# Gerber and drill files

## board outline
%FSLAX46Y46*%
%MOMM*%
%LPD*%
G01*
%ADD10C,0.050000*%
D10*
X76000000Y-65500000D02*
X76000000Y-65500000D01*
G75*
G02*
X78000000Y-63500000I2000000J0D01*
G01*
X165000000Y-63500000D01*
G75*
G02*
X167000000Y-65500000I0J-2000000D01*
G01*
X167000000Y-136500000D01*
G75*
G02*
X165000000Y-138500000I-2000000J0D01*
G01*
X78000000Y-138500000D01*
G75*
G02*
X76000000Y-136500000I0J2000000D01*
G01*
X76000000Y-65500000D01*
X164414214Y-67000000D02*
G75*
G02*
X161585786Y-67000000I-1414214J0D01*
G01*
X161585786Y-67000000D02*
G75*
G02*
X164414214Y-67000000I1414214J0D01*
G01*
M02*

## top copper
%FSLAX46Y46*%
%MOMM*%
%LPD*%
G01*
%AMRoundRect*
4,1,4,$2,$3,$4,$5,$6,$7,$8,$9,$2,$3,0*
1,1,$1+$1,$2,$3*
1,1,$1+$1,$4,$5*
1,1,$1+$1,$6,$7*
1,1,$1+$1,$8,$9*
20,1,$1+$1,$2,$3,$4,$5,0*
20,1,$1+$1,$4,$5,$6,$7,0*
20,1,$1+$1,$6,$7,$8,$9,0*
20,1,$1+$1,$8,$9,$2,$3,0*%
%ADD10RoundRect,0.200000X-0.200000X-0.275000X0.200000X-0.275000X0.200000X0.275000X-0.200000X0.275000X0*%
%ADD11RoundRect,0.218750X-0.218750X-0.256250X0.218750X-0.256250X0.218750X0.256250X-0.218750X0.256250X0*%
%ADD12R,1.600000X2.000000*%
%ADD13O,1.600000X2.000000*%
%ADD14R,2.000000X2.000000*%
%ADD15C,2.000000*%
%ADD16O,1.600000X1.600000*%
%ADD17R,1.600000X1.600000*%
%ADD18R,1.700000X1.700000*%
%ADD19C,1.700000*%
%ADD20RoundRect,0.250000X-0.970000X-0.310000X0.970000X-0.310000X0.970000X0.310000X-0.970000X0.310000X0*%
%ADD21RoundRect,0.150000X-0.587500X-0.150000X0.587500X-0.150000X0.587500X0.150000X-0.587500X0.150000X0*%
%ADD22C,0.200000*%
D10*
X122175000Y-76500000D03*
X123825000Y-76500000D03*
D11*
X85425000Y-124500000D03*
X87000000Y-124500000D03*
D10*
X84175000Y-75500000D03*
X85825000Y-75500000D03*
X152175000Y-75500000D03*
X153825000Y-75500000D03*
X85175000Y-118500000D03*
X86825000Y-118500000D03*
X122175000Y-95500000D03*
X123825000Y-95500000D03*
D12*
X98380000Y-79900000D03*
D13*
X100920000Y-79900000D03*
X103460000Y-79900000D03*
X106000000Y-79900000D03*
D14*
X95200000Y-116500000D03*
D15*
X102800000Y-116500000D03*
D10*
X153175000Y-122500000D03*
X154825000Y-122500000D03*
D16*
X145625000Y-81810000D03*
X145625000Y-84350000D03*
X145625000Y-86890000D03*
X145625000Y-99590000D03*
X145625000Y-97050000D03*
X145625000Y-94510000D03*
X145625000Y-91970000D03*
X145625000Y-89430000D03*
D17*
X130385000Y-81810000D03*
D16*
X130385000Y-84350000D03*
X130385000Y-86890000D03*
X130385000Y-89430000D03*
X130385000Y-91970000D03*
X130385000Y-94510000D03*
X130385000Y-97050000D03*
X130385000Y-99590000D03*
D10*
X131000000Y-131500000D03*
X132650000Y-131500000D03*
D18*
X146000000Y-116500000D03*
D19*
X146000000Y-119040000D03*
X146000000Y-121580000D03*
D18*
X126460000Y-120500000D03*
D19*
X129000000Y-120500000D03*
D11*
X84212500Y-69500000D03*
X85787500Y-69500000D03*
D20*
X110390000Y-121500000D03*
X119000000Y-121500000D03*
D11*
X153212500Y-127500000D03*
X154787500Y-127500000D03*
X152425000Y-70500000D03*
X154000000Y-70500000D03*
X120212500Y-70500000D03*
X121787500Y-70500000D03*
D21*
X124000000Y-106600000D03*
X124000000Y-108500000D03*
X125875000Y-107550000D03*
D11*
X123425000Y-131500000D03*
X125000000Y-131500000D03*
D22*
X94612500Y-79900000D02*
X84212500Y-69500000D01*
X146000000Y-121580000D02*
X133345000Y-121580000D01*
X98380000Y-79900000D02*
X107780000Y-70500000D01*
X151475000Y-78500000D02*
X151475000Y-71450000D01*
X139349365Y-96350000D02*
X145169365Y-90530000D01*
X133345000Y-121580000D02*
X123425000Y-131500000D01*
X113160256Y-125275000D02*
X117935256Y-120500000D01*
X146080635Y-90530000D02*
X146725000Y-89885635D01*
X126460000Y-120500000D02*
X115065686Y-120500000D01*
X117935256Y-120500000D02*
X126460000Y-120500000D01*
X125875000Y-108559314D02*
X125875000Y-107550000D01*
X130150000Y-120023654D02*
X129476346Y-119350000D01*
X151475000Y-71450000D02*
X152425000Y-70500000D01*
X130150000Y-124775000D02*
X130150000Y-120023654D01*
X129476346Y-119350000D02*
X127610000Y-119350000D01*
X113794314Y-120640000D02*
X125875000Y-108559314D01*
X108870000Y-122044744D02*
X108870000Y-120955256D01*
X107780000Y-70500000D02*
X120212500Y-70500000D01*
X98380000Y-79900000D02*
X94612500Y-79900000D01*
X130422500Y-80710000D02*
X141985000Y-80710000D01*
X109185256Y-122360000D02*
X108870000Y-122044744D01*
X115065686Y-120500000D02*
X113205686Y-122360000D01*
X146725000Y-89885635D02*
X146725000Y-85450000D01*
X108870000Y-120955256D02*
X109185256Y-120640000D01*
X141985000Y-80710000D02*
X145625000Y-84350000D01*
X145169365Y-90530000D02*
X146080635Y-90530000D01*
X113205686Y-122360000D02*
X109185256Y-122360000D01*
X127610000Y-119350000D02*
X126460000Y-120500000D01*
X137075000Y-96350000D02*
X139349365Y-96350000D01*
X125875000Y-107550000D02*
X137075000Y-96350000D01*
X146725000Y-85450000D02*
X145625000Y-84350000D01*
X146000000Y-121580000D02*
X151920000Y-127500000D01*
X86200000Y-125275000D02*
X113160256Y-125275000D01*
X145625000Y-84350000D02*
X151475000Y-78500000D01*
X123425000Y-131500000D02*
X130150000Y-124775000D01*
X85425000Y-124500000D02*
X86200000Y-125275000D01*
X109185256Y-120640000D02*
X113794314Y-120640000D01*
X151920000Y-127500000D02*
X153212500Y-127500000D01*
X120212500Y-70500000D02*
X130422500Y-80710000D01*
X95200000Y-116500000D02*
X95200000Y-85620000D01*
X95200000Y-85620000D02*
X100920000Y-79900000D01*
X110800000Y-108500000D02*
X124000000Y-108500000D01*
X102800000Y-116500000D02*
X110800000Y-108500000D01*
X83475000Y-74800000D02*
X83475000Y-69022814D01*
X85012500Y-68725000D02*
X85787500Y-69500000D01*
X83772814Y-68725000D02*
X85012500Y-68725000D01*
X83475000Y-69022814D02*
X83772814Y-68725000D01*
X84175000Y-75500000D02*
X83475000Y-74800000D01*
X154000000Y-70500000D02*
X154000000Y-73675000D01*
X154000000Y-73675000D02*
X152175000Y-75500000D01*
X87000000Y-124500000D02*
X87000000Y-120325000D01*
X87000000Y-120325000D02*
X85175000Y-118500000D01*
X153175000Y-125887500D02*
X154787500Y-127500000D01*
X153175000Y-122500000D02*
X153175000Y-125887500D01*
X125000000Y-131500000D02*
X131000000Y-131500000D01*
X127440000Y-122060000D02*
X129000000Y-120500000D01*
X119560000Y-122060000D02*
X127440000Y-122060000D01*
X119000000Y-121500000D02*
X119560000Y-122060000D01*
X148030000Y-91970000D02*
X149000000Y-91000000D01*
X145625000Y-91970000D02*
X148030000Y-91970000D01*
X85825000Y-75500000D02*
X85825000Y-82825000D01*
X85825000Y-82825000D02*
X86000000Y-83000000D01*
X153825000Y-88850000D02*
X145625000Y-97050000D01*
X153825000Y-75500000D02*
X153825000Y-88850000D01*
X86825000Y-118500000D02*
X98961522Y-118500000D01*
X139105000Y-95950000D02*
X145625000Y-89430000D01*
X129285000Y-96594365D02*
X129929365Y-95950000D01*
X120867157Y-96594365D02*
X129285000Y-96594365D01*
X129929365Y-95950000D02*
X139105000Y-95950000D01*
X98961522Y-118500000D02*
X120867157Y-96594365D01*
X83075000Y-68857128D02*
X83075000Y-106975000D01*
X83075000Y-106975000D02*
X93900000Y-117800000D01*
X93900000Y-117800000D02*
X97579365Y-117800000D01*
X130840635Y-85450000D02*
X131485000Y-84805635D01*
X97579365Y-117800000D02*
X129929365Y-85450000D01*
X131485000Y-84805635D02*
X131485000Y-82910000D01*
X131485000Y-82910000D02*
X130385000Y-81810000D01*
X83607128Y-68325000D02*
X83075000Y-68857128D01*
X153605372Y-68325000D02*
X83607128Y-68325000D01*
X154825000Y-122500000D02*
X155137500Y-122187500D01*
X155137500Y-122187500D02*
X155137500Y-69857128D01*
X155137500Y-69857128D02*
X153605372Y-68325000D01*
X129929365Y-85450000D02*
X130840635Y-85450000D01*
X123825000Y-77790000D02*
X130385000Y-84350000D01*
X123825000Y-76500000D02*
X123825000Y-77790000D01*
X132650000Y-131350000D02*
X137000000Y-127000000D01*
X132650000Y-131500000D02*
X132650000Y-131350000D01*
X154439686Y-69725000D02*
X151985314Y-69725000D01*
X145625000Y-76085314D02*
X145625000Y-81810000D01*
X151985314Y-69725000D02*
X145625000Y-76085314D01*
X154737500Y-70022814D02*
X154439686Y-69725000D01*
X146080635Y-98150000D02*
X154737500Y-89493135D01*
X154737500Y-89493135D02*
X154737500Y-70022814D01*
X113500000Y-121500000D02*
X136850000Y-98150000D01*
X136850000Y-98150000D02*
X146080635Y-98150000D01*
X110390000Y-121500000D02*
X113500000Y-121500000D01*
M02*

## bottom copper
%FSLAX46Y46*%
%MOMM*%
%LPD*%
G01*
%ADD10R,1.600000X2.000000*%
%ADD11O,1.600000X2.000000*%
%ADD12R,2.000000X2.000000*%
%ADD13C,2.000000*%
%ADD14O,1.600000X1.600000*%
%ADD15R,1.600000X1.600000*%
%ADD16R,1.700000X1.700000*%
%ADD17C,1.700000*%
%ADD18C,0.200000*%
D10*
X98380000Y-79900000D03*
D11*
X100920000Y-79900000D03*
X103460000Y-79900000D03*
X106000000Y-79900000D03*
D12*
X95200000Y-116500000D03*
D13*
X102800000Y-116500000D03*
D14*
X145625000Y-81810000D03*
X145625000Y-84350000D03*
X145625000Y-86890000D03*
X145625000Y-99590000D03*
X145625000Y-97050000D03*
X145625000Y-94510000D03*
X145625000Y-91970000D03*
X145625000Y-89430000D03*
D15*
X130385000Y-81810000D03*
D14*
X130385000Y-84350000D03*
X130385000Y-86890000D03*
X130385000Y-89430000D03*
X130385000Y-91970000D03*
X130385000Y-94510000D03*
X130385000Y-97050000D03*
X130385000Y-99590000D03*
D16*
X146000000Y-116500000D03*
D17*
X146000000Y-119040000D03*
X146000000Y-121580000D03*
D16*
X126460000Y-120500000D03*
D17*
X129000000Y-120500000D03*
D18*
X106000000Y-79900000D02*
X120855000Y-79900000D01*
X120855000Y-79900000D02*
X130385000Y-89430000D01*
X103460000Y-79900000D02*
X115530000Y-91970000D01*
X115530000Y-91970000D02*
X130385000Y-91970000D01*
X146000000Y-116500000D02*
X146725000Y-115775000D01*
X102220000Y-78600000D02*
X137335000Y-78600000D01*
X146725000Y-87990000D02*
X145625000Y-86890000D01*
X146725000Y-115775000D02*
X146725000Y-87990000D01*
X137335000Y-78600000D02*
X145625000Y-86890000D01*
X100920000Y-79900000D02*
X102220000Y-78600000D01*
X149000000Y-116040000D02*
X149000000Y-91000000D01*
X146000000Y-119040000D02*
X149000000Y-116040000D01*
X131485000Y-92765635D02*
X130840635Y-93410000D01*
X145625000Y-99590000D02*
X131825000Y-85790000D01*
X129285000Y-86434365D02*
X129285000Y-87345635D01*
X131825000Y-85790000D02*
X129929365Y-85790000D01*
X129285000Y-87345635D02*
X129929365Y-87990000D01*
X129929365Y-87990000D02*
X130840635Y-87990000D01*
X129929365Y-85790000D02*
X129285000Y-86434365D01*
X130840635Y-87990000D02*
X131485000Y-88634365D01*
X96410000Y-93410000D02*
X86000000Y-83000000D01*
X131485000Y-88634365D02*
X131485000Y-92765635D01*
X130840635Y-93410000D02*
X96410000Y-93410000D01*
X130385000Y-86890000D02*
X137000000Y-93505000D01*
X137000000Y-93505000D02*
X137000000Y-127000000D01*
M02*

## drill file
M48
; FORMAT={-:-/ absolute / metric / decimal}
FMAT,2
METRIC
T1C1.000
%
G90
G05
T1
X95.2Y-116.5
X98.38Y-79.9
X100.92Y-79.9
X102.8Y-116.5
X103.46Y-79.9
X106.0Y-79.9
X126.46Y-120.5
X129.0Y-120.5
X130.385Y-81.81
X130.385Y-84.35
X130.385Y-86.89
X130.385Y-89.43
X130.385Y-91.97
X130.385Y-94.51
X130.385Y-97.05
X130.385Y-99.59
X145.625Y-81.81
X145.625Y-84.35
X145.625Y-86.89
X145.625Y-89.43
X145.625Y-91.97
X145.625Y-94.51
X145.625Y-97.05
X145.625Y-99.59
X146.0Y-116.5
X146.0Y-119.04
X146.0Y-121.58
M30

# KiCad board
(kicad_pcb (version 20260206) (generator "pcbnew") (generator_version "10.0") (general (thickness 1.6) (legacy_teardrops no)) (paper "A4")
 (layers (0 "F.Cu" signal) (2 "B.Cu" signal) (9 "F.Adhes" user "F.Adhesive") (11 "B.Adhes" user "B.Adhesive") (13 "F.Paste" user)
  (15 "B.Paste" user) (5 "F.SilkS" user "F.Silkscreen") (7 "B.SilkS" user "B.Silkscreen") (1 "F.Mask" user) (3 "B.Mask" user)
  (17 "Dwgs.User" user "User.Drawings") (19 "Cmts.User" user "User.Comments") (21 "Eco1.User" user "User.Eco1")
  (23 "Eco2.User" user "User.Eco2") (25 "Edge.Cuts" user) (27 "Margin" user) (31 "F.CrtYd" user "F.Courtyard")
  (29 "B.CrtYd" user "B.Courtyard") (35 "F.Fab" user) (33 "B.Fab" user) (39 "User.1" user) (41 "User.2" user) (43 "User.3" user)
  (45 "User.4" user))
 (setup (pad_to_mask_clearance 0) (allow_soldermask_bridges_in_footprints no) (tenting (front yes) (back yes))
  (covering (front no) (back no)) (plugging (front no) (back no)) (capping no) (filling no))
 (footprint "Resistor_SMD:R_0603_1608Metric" (layer "F.Cu") (at 123 76.5)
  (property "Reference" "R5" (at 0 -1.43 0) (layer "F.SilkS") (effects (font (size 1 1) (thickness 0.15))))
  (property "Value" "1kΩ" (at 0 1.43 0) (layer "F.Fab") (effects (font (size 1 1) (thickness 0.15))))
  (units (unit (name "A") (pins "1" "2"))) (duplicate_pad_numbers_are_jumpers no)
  (pad "1" smd roundrect (at -0.825 0) (size 0.8 0.95) (layers "F.Cu" "F.Mask" "F.Paste") (roundrect_rratio 0.25) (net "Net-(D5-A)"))
  (pad "2" smd roundrect (at 0.825 0) (size 0.8 0.95) (layers "F.Cu" "F.Mask" "F.Paste") (roundrect_rratio 0.25) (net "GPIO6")))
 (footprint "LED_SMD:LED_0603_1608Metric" (layer "F.Cu") (at 86.2125 124.5)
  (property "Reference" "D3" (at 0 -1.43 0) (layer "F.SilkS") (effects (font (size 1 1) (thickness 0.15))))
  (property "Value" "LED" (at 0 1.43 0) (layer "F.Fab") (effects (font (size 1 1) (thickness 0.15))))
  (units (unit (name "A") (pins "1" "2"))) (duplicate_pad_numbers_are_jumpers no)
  (pad "1" smd roundrect (at -0.7875 0) (size 0.875 0.95) (layers "F.Cu" "F.Mask" "F.Paste") (roundrect_rratio 0.25) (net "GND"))
  (pad "2" smd roundrect (at 0.7875 0) (size 0.875 0.95) (layers "F.Cu" "F.Mask" "F.Paste") (roundrect_rratio 0.25) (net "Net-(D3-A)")))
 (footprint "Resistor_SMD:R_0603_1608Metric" (layer "F.Cu") (at 85 75.5)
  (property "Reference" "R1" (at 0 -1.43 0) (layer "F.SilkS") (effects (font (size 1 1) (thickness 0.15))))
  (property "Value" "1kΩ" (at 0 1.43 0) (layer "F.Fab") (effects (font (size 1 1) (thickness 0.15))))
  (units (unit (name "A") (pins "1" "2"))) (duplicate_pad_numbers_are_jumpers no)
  (pad "1" smd roundrect (at -0.825 0) (size 0.8 0.95) (layers "F.Cu" "F.Mask" "F.Paste") (roundrect_rratio 0.25) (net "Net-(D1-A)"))
  (pad "2" smd roundrect (at 0.825 0) (size 0.8 0.95) (layers "F.Cu" "F.Mask" "F.Paste") (roundrect_rratio 0.25) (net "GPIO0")))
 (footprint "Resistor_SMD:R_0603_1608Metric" (layer "F.Cu") (at 153 75.5)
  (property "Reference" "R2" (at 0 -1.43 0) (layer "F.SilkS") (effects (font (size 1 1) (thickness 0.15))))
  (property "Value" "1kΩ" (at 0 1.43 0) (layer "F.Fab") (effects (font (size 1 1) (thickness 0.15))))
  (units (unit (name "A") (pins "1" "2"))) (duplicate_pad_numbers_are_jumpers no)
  (pad "1" smd roundrect (at -0.825 0) (size 0.8 0.95) (layers "F.Cu" "F.Mask" "F.Paste") (roundrect_rratio 0.25) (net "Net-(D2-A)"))
  (pad "2" smd roundrect (at 0.825 0) (size 0.8 0.95) (layers "F.Cu" "F.Mask" "F.Paste") (roundrect_rratio 0.25) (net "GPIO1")))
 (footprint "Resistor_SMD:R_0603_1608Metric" (layer "F.Cu") (at 86 118.5)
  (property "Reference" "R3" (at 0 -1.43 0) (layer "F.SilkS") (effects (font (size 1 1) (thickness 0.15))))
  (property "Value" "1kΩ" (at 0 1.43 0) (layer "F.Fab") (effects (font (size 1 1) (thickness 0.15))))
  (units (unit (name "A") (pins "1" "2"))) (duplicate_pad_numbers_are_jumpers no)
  (pad "1" smd roundrect (at -0.825 0) (size 0.8 0.95) (layers "F.Cu" "F.Mask" "F.Paste") (roundrect_rratio 0.25) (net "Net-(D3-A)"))
  (pad "2" smd roundrect (at 0.825 0) (size 0.8 0.95) (layers "F.Cu" "F.Mask" "F.Paste") (roundrect_rratio 0.25) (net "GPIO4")))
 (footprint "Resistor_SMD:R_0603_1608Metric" (layer "F.Cu") (at 123 95.5)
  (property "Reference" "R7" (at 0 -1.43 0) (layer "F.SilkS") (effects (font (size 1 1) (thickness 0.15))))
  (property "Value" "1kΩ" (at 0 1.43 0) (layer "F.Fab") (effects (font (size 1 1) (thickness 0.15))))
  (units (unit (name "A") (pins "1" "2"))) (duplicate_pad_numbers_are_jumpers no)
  (pad "1" smd roundrect (at -0.825 0) (size 0.8 0.95) (layers "F.Cu" "F.Mask" "F.Paste") (roundrect_rratio 0.25) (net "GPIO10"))
  (pad "2" smd roundrect (at 0.825 0) (size 0.8 0.95) (layers "F.Cu" "F.Mask" "F.Paste") (roundrect_rratio 0.25) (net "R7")))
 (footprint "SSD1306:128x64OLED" (layer "F.Cu") (at 102 90.5)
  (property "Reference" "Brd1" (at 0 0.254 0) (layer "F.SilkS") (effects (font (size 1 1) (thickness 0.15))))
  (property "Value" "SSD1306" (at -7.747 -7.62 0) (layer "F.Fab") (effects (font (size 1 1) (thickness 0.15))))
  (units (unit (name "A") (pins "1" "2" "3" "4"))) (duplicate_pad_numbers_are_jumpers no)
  (pad "1" thru_hole rect (at -3.62 -10.6 90) (size 2 1.6) (drill 1) (layers "*.Cu" "*.Mask") (remove_unused_layers no) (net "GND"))
  (pad "2" thru_hole oval (at -1.08 -10.6 90) (size 2 1.6) (drill 1) (layers "*.Cu" "*.Mask") (remove_unused_layers no) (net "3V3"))
  (pad "3" thru_hole oval (at 1.46 -10.6 90) (size 2 1.6) (drill 1) (layers "*.Cu" "*.Mask") (remove_unused_layers no) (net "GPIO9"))
  (pad "4" thru_hole oval (at 4 -10.6 90) (size 2 1.6) (drill 1) (layers "*.Cu" "*.Mask") (remove_unused_layers no) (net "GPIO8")))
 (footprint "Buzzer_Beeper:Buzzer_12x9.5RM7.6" (layer "F.Cu") (at 95.2 116.5)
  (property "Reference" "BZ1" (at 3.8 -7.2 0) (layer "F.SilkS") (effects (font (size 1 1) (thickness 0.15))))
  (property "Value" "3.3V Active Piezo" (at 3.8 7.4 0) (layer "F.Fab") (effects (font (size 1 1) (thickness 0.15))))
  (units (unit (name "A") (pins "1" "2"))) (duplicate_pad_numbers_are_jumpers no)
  (pad "1" thru_hole rect (at 0 0) (size 2 2) (drill 1) (layers "*.Cu" "*.Mask") (remove_unused_layers no) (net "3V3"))
  (pad "2" thru_hole circle (at 7.6 0) (size 2 2) (drill 1) (layers "*.Cu" "*.Mask") (remove_unused_layers no) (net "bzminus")))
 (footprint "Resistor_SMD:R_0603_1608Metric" (layer "F.Cu") (at 154 122.5)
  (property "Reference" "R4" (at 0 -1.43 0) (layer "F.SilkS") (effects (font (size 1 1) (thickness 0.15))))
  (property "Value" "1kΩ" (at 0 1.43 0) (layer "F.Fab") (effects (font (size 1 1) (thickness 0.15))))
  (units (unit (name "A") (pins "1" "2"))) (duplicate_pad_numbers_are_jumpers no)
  (pad "1" smd roundrect (at -0.825 0) (size 0.8 0.95) (layers "F.Cu" "F.Mask" "F.Paste") (roundrect_rratio 0.25) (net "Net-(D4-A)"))
  (pad "2" smd roundrect (at 0.825 0) (size 0.8 0.95) (layers "F.Cu" "F.Mask" "F.Paste") (roundrect_rratio 0.25) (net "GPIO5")))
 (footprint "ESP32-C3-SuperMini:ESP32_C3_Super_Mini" (layer "F.Cu") (at 130.385 81.81)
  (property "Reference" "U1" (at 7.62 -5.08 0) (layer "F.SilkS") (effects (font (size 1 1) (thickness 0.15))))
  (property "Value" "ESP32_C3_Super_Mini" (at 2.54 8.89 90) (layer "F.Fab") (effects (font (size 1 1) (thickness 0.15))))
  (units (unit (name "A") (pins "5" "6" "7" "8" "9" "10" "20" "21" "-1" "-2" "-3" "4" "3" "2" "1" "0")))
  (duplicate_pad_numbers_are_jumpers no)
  (pad "-1" thru_hole oval (at 15.24 0) (size 1.6 1.6) (drill 1) (layers "*.Cu" "*.Mask") (remove_unused_layers no) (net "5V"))
  (pad "-2" thru_hole oval (at 15.24 2.54) (size 1.6 1.6) (drill 1) (layers "*.Cu" "*.Mask") (remove_unused_layers no) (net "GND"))
  (pad "-3" thru_hole oval (at 15.24 5.08) (size 1.6 1.6) (drill 1) (layers "*.Cu" "*.Mask") (remove_unused_layers no) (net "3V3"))
  (pad "0" thru_hole oval (at 15.24 17.78) (size 1.6 1.6) (drill 1) (layers "*.Cu" "*.Mask") (remove_unused_layers no) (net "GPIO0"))
  (pad "1" thru_hole oval (at 15.24 15.24) (size 1.6 1.6) (drill 1) (layers "*.Cu" "*.Mask") (remove_unused_layers no) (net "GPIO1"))
  (pad "2" thru_hole oval (at 15.24 12.7) (size 1.6 1.6) (drill 1) (layers "*.Cu" "*.Mask") (remove_unused_layers no)
   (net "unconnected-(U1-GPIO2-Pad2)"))
  (pad "3" thru_hole oval (at 15.24 10.16) (size 1.6 1.6) (drill 1) (layers "*.Cu" "*.Mask") (remove_unused_layers no) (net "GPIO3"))
  (pad "4" thru_hole oval (at 15.24 7.62) (size 1.6 1.6) (drill 1) (layers "*.Cu" "*.Mask") (remove_unused_layers no) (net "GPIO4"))
  (pad "5" thru_hole rect (at 0 0) (size 1.6 1.6) (drill 1) (layers "*.Cu" "*.Mask") (remove_unused_layers no) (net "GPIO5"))
  (pad "6" thru_hole oval (at 0 2.54) (size 1.6 1.6) (drill 1) (layers "*.Cu" "*.Mask") (remove_unused_layers no) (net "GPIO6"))
  (pad "7" thru_hole oval (at 0 5.08) (size 1.6 1.6) (drill 1) (layers "*.Cu" "*.Mask") (remove_unused_layers no) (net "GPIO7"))
  (pad "8" thru_hole oval (at 0 7.62) (size 1.6 1.6) (drill 1) (layers "*.Cu" "*.Mask") (remove_unused_layers no) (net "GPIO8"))
  (pad "9" thru_hole oval (at 0 10.16) (size 1.6 1.6) (drill 1) (layers "*.Cu" "*.Mask") (remove_unused_layers no) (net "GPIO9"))
  (pad "10" thru_hole oval (at 0 12.7) (size 1.6 1.6) (drill 1) (layers "*.Cu" "*.Mask") (remove_unused_layers no) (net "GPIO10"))
  (pad "20" thru_hole oval (at 0 15.24) (size 1.6 1.6) (drill 1) (layers "*.Cu" "*.Mask") (remove_unused_layers no)
   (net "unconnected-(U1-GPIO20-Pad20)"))
  (pad "21" thru_hole oval (at 0 17.78) (size 1.6 1.6) (drill 1) (layers "*.Cu" "*.Mask") (remove_unused_layers no)
   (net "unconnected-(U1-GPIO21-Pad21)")))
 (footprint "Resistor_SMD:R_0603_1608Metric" (layer "F.Cu") (at 131.825 131.5)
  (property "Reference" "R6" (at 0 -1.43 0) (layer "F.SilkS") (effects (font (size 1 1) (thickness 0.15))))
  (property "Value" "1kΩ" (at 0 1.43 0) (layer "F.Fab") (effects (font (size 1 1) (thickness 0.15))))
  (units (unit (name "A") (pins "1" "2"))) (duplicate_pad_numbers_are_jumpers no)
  (pad "1" smd roundrect (at -0.825 0) (size 0.8 0.95) (layers "F.Cu" "F.Mask" "F.Paste") (roundrect_rratio 0.25) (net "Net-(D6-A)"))
  (pad "2" smd roundrect (at 0.825 0) (size 0.8 0.95) (layers "F.Cu" "F.Mask" "F.Paste") (roundrect_rratio 0.25) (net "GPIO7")))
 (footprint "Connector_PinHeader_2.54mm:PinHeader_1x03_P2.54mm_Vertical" (layer "F.Cu") (at 146 116.5)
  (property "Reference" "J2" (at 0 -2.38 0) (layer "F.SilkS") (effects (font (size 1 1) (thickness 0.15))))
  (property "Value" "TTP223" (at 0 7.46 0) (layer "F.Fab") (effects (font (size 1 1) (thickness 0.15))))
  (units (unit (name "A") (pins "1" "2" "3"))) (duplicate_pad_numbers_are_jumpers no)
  (pad "1" thru_hole rect (at 0 0) (size 1.7 1.7) (drill 1) (layers "*.Cu" "*.Mask") (remove_unused_layers no) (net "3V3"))
  (pad "2" thru_hole circle (at 0 2.54) (size 1.7 1.7) (drill 1) (layers "*.Cu" "*.Mask") (remove_unused_layers no) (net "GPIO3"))
  (pad "3" thru_hole circle (at 0 5.08) (size 1.7 1.7) (drill 1) (layers "*.Cu" "*.Mask") (remove_unused_layers no) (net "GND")))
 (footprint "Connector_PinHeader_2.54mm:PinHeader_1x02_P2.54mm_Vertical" (layer "F.Cu") (at 126.46 120.5 90)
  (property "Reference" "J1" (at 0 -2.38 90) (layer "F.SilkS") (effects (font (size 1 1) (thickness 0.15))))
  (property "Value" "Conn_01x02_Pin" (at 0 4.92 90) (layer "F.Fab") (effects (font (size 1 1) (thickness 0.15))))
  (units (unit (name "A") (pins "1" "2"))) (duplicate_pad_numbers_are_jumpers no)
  (pad "1" thru_hole rect (at 0 0 90) (size 1.7 1.7) (drill 1) (layers "*.Cu" "*.Mask") (remove_unused_layers no) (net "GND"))
  (pad "2" thru_hole circle (at 0 2.54 90) (size 1.7 1.7) (drill 1) (layers "*.Cu" "*.Mask") (remove_unused_layers no)
   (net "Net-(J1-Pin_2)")))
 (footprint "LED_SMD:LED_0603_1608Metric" (layer "F.Cu") (at 85 69.5)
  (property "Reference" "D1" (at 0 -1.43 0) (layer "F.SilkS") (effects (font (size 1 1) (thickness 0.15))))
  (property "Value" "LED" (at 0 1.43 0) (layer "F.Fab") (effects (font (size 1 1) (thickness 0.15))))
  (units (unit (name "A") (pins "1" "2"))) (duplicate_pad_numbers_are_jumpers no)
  (pad "1" smd roundrect (at -0.7875 0) (size 0.875 0.95) (layers "F.Cu" "F.Mask" "F.Paste") (roundrect_rratio 0.25) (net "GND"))
  (pad "2" smd roundrect (at 0.7875 0) (size 0.875 0.95) (layers "F.Cu" "F.Mask" "F.Paste") (roundrect_rratio 0.25) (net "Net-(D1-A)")))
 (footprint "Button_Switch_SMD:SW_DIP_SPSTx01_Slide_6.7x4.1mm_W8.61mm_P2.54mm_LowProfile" (layer "F.Cu") (at 114.695 121.5)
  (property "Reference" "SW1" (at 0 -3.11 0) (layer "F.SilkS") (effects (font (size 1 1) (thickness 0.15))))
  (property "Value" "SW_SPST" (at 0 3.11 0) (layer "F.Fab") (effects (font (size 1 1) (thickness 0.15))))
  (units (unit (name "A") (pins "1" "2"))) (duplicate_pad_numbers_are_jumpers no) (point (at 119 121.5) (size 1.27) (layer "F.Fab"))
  (pad "1" smd roundrect (at -4.305 0) (size 2.44 1.12) (layers "F.Cu" "F.Mask" "F.Paste") (roundrect_rratio 0.223214) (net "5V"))
  (pad "2" smd roundrect (at 4.305 0) (size 2.44 1.12) (layers "F.Cu" "F.Mask" "F.Paste") (roundrect_rratio 0.223214) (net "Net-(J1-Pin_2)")))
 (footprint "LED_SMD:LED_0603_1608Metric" (layer "F.Cu") (at 154 127.5)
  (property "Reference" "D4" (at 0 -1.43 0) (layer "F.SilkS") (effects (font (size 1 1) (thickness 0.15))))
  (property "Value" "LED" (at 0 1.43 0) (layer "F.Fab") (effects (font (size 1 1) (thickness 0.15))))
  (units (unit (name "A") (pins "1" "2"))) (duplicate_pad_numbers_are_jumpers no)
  (pad "1" smd roundrect (at -0.7875 0) (size 0.875 0.95) (layers "F.Cu" "F.Mask" "F.Paste") (roundrect_rratio 0.25) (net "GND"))
  (pad "2" smd roundrect (at 0.7875 0) (size 0.875 0.95) (layers "F.Cu" "F.Mask" "F.Paste") (roundrect_rratio 0.25) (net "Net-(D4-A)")))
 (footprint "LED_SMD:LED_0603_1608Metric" (layer "F.Cu") (at 153.2125 70.5)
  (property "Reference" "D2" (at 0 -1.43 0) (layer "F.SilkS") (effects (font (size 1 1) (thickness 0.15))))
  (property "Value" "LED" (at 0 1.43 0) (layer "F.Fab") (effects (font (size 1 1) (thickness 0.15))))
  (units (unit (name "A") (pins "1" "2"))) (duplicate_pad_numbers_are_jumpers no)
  (pad "1" smd roundrect (at -0.7875 0) (size 0.875 0.95) (layers "F.Cu" "F.Mask" "F.Paste") (roundrect_rratio 0.25) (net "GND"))
  (pad "2" smd roundrect (at 0.7875 0) (size 0.875 0.95) (layers "F.Cu" "F.Mask" "F.Paste") (roundrect_rratio 0.25) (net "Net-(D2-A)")))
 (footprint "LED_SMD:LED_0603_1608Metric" (layer "F.Cu") (at 121 70.5)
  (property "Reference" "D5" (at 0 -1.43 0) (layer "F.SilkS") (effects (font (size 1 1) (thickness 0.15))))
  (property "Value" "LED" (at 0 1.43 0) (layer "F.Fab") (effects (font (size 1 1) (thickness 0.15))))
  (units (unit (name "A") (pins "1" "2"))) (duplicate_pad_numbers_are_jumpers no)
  (pad "1" smd roundrect (at -0.7875 0) (size 0.875 0.95) (layers "F.Cu" "F.Mask" "F.Paste") (roundrect_rratio 0.25) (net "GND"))
  (pad "2" smd roundrect (at 0.7875 0) (size 0.875 0.95) (layers "F.Cu" "F.Mask" "F.Paste") (roundrect_rratio 0.25) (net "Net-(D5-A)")))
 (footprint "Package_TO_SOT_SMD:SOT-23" (layer "F.Cu") (at 124.9375 107.55)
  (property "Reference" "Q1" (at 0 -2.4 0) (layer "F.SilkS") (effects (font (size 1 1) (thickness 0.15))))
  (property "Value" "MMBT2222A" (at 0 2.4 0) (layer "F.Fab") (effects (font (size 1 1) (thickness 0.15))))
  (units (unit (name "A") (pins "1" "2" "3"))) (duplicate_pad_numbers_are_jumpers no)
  (pad "1" smd roundrect (at -0.9375 -0.95) (size 1.475 0.6) (layers "F.Cu" "F.Mask" "F.Paste") (roundrect_rratio 0.25) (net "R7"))
  (pad "2" smd roundrect (at -0.9375 0.95) (size 1.475 0.6) (layers "F.Cu" "F.Mask" "F.Paste") (roundrect_rratio 0.25) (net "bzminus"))
  (pad "3" smd roundrect (at 0.9375 0) (size 1.475 0.6) (layers "F.Cu" "F.Mask" "F.Paste") (roundrect_rratio 0.25) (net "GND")))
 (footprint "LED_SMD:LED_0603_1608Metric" (layer "F.Cu") (at 124.2125 131.5)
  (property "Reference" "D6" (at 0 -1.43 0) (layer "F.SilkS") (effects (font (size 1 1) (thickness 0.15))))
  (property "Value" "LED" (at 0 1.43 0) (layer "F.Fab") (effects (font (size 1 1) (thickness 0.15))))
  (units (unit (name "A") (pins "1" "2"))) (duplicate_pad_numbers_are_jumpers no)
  (pad "1" smd roundrect (at -0.7875 0) (size 0.875 0.95) (layers "F.Cu" "F.Mask" "F.Paste") (roundrect_rratio 0.25) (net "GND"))
  (pad "2" smd roundrect (at 0.7875 0) (size 0.875 0.95) (layers "F.Cu" "F.Mask" "F.Paste") (roundrect_rratio 0.25) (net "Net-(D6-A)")))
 (gr_rect (start 76 63.5) (end 167 138.5) (radius 2) (stroke (width 0.05) (type default)) (fill no) (layer "Edge.Cuts"))
 (gr_circle (center 163 67) (end 164 68) (stroke (width 0.05) (type default)) (fill no) (layer "Edge.Cuts"))
 (segment (start 94.6125 79.9) (end 84.2125 69.5) (width 0.2) (layer "F.Cu") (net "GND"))
 (segment (start 146 121.58) (end 133.345 121.58) (width 0.2) (layer "F.Cu") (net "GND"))
 (segment (start 98.38 79.9) (end 107.78 70.5) (width 0.2) (layer "F.Cu") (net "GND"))
 (segment (start 151.475 78.5) (end 151.475 71.45) (width 0.2) (layer "F.Cu") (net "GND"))
 (segment (start 139.349365 96.35) (end 145.169365 90.53) (width 0.2) (layer "F.Cu") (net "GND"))
 (segment (start 133.345 121.58) (end 123.425 131.5) (width 0.2) (layer "F.Cu") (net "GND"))
 (segment (start 113.160256 125.275) (end 117.935256 120.5) (width 0.2) (layer "F.Cu") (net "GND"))
 (segment (start 146.080635 90.53) (end 146.725 89.885635) (width 0.2) (layer "F.Cu") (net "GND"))
 (segment (start 126.46 120.5) (end 115.065686 120.5) (width 0.2) (layer "F.Cu") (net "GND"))
 (segment (start 117.935256 120.5) (end 126.46 120.5) (width 0.2) (layer "F.Cu") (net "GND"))
 (segment (start 125.875 108.559314) (end 125.875 107.55) (width 0.2) (layer "F.Cu") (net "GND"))
 (segment (start 130.15 120.023654) (end 129.476346 119.35) (width 0.2) (layer "F.Cu") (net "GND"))
 (segment (start 151.475 71.45) (end 152.425 70.5) (width 0.2) (layer "F.Cu") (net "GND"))
 (segment (start 130.15 124.775) (end 130.15 120.023654) (width 0.2) (layer "F.Cu") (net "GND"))
 (segment (start 129.476346 119.35) (end 127.61 119.35) (width 0.2) (layer "F.Cu") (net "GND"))
 (segment (start 113.794314 120.64) (end 125.875 108.559314) (width 0.2) (layer "F.Cu") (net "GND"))
 (segment (start 108.87 122.044744) (end 108.87 120.955256) (width 0.2) (layer "F.Cu") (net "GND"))
 (segment (start 107.78 70.5) (end 120.2125 70.5) (width 0.2) (layer "F.Cu") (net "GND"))
 (segment (start 98.38 79.9) (end 94.6125 79.9) (width 0.2) (layer "F.Cu") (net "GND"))
 (segment (start 130.4225 80.71) (end 141.985 80.71) (width 0.2) (layer "F.Cu") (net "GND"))
 (segment (start 109.185256 122.36) (end 108.87 122.044744) (width 0.2) (layer "F.Cu") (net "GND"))
 (segment (start 115.065686 120.5) (end 113.205686 122.36) (width 0.2) (layer "F.Cu") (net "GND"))
 (segment (start 146.725 89.885635) (end 146.725 85.45) (width 0.2) (layer "F.Cu") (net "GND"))
 (segment (start 108.87 120.955256) (end 109.185256 120.64) (width 0.2) (layer "F.Cu") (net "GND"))
 (segment (start 141.985 80.71) (end 145.625 84.35) (width 0.2) (layer "F.Cu") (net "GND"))
 (segment (start 145.169365 90.53) (end 146.080635 90.53) (width 0.2) (layer "F.Cu") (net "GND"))
 (segment (start 113.205686 122.36) (end 109.185256 122.36) (width 0.2) (layer "F.Cu") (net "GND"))
 (segment (start 127.61 119.35) (end 126.46 120.5) (width 0.2) (layer "F.Cu") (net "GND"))
 (segment (start 137.075 96.35) (end 139.349365 96.35) (width 0.2) (layer "F.Cu") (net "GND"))
 (segment (start 125.875 107.55) (end 137.075 96.35) (width 0.2) (layer "F.Cu") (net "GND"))
 (segment (start 146.725 85.45) (end 145.625 84.35) (width 0.2) (layer "F.Cu") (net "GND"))
 (segment (start 146 121.58) (end 151.92 127.5) (width 0.2) (layer "F.Cu") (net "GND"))
 (segment (start 86.2 125.275) (end 113.160256 125.275) (width 0.2) (layer "F.Cu") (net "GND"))
 (segment (start 145.625 84.35) (end 151.475 78.5) (width 0.2) (layer "F.Cu") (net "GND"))
 (segment (start 123.425 131.5) (end 130.15 124.775) (width 0.2) (layer "F.Cu") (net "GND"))
 (segment (start 85.425 124.5) (end 86.2 125.275) (width 0.2) (layer "F.Cu") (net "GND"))
 (segment (start 109.185256 120.64) (end 113.794314 120.64) (width 0.2) (layer "F.Cu") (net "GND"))
 (segment (start 151.92 127.5) (end 153.2125 127.5) (width 0.2) (layer "F.Cu") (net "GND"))
 (segment (start 120.2125 70.5) (end 130.4225 80.71) (width 0.2) (layer "F.Cu") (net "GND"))
 (segment (start 106 79.9) (end 120.855 79.9) (width 0.2) (layer "B.Cu") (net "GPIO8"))
 (segment (start 120.855 79.9) (end 130.385 89.43) (width 0.2) (layer "B.Cu") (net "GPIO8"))
 (segment (start 103.46 79.9) (end 115.53 91.97) (width 0.2) (layer "B.Cu") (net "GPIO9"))
 (segment (start 115.53 91.97) (end 130.385 91.97) (width 0.2) (layer "B.Cu") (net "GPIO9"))
 (segment (start 95.2 116.5) (end 95.2 85.62) (width 0.2) (layer "F.Cu") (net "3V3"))
 (segment (start 95.2 85.62) (end 100.92 79.9) (width 0.2) (layer "F.Cu") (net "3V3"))
 (segment (start 146 116.5) (end 146.725 115.775) (width 0.2) (layer "B.Cu") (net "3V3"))
 (segment (start 102.22 78.6) (end 137.335 78.6) (width 0.2) (layer "B.Cu") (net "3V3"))
 (segment (start 146.725 87.99) (end 145.625 86.89) (width 0.2) (layer "B.Cu") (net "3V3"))
 (segment (start 146.725 115.775) (end 146.725 87.99) (width 0.2) (layer "B.Cu") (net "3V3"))
 (segment (start 137.335 78.6) (end 145.625 86.89) (width 0.2) (layer "B.Cu") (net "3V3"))
 (segment (start 100.92 79.9) (end 102.22 78.6) (width 0.2) (layer "B.Cu") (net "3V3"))
 (segment (start 110.8 108.5) (end 124 108.5) (width 0.2) (layer "F.Cu") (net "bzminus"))
 (segment (start 102.8 116.5) (end 110.8 108.5) (width 0.2) (layer "F.Cu") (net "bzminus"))
 (segment (start 83.475 74.8) (end 83.475 69.022814) (width 0.2) (layer "F.Cu") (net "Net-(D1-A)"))
 (segment (start 85.0125 68.725) (end 85.7875 69.5) (width 0.2) (layer "F.Cu") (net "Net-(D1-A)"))
 (segment (start 83.772814 68.725) (end 85.0125 68.725) (width 0.2) (layer "F.Cu") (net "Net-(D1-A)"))
 (segment (start 83.475 69.022814) (end 83.772814 68.725) (width 0.2) (layer "F.Cu") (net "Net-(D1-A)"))
 (segment (start 84.175 75.5) (end 83.475 74.8) (width 0.2) (layer "F.Cu") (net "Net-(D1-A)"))
 (segment (start 154 70.5) (end 154 73.675) (width 0.2) (layer "F.Cu") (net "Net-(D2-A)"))
 (segment (start 154 73.675) (end 152.175 75.5) (width 0.2) (layer "F.Cu") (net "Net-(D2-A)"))
 (segment (start 87 124.5) (end 87 120.325) (width 0.2) (layer "F.Cu") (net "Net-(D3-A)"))
 (segment (start 87 120.325) (end 85.175 118.5) (width 0.2) (layer "F.Cu") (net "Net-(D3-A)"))
 (segment (start 153.175 125.8875) (end 154.7875 127.5) (width 0.2) (layer "F.Cu") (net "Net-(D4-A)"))
 (segment (start 153.175 122.5) (end 153.175 125.8875) (width 0.2) (layer "F.Cu") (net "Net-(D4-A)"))
 (segment (start 125 131.5) (end 131 131.5) (width 0.2) (layer "F.Cu") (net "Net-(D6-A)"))
 (segment (start 127.44 122.06) (end 129 120.5) (width 0.2) (layer "F.Cu") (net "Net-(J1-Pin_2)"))
 (segment (start 119.56 122.06) (end 127.44 122.06) (width 0.2) (layer "F.Cu") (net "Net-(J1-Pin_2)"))
 (segment (start 119 121.5) (end 119.56 122.06) (width 0.2) (layer "F.Cu") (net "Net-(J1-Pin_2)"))
 (segment (start 148.03 91.97) (end 149 91) (width 0.2) (layer "F.Cu") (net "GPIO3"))
 (segment (start 145.625 91.97) (end 148.03 91.97) (width 0.2) (layer "F.Cu") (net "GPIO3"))
 (segment (start 149 116.04) (end 149 91) (width 0.2) (layer "B.Cu") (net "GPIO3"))
 (segment (start 146 119.04) (end 149 116.04) (width 0.2) (layer "B.Cu") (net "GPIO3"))
 (segment (start 85.825 75.5) (end 85.825 82.825) (width 0.2) (layer "F.Cu") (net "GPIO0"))
 (segment (start 85.825 82.825) (end 86 83) (width 0.2) (layer "F.Cu") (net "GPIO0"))
 (segment (start 131.485 92.765635) (end 130.840635 93.41) (width 0.2) (layer "B.Cu") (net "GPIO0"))
 (segment (start 145.625 99.59) (end 131.825 85.79) (width 0.2) (layer "B.Cu") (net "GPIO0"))
 (segment (start 129.285 86.434365) (end 129.285 87.345635) (width 0.2) (layer "B.Cu") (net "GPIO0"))
 (segment (start 131.825 85.79) (end 129.929365 85.79) (width 0.2) (layer "B.Cu") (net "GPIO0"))
 (segment (start 129.285 87.345635) (end 129.929365 87.99) (width 0.2) (layer "B.Cu") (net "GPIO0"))
 (segment (start 129.929365 87.99) (end 130.840635 87.99) (width 0.2) (layer "B.Cu") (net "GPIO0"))
 (segment (start 129.929365 85.79) (end 129.285 86.434365) (width 0.2) (layer "B.Cu") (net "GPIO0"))
 (segment (start 130.840635 87.99) (end 131.485 88.634365) (width 0.2) (layer "B.Cu") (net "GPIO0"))
 (segment (start 96.41 93.41) (end 86 83) (width 0.2) (layer "B.Cu") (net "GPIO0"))
 (segment (start 131.485 88.634365) (end 131.485 92.765635) (width 0.2) (layer "B.Cu") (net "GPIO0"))
 (segment (start 130.840635 93.41) (end 96.41 93.41) (width 0.2) (layer "B.Cu") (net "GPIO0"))
 (segment (start 153.825 88.85) (end 145.625 97.05) (width 0.2) (layer "F.Cu") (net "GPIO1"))
 (segment (start 153.825 75.5) (end 153.825 88.85) (width 0.2) (layer "F.Cu") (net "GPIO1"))
 (segment (start 86.825 118.5) (end 98.961522 118.5) (width 0.2) (layer "F.Cu") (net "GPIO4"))
 (segment (start 139.105 95.95) (end 145.625 89.43) (width 0.2) (layer "F.Cu") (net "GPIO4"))
 (segment (start 129.285 96.594365) (end 129.929365 95.95) (width 0.2) (layer "F.Cu") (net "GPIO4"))
 (segment (start 120.867157 96.594365) (end 129.285 96.594365) (width 0.2) (layer "F.Cu") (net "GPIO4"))
 (segment (start 129.929365 95.95) (end 139.105 95.95) (width 0.2) (layer "F.Cu") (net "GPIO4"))
 (segment (start 98.961522 118.5) (end 120.867157 96.594365) (width 0.2) (layer "F.Cu") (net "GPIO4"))
 (segment (start 83.075 68.857128) (end 83.075 106.975) (width 0.2) (layer "F.Cu") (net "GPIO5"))
 (segment (start 83.075 106.975) (end 93.9 117.8) (width 0.2) (layer "F.Cu") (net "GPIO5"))
 (segment (start 93.9 117.8) (end 97.579365 117.8) (width 0.2) (layer "F.Cu") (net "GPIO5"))
 (segment (start 130.840635 85.45) (end 131.485 84.805635) (width 0.2) (layer "F.Cu") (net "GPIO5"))
 (segment (start 97.579365 117.8) (end 129.929365 85.45) (width 0.2) (layer "F.Cu") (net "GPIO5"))
 (segment (start 131.485 84.805635) (end 131.485 82.91) (width 0.2) (layer "F.Cu") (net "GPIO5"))
 (segment (start 131.485 82.91) (end 130.385 81.81) (width 0.2) (layer "F.Cu") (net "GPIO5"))
 (segment (start 83.607128 68.325) (end 83.075 68.857128) (width 0.2) (layer "F.Cu") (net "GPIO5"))
 (segment (start 153.605372 68.325) (end 83.607128 68.325) (width 0.2) (layer "F.Cu") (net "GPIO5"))
 (segment (start 154.825 122.5) (end 155.1375 122.1875) (width 0.2) (layer "F.Cu") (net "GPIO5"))
 (segment (start 155.1375 122.1875) (end 155.1375 69.857128) (width 0.2) (layer "F.Cu") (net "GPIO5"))
 (segment (start 155.1375 69.857128) (end 153.605372 68.325) (width 0.2) (layer "F.Cu") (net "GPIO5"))
 (segment (start 129.929365 85.45) (end 130.840635 85.45) (width 0.2) (layer "F.Cu") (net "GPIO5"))
 (segment (start 123.825 77.79) (end 130.385 84.35) (width 0.2) (layer "F.Cu") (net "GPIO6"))
 (segment (start 123.825 76.5) (end 123.825 77.79) (width 0.2) (layer "F.Cu") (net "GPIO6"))
 (segment (start 132.65 131.35) (end 137 127) (width 0.2) (layer "F.Cu") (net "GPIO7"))
 (segment (start 132.65 131.5) (end 132.65 131.35) (width 0.2) (layer "F.Cu") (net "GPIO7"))
 (segment (start 130.385 86.89) (end 137 93.505) (width 0.2) (layer "B.Cu") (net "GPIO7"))
 (segment (start 137 93.505) (end 137 127) (width 0.2) (layer "B.Cu") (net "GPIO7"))
 (segment (start 154.439686 69.725) (end 151.985314 69.725) (width 0.2) (layer "F.Cu") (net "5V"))
 (segment (start 145.625 76.085314) (end 145.625 81.81) (width 0.2) (layer "F.Cu") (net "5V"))
 (segment (start 151.985314 69.725) (end 145.625 76.085314) (width 0.2) (layer "F.Cu") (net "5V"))
 (segment (start 154.7375 70.022814) (end 154.439686 69.725) (width 0.2) (layer "F.Cu") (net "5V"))
 (segment (start 146.080635 98.15) (end 154.7375 89.493135) (width 0.2) (layer "F.Cu") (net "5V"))
 (segment (start 154.7375 89.493135) (end 154.7375 70.022814) (width 0.2) (layer "F.Cu") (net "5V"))
 (segment (start 113.5 121.5) (end 136.85 98.15) (width 0.2) (layer "F.Cu") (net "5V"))
 (segment (start 136.85 98.15) (end 146.080635 98.15) (width 0.2) (layer "F.Cu") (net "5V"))
 (segment (start 110.39 121.5) (end 113.5 121.5) (width 0.2) (layer "F.Cu") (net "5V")))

